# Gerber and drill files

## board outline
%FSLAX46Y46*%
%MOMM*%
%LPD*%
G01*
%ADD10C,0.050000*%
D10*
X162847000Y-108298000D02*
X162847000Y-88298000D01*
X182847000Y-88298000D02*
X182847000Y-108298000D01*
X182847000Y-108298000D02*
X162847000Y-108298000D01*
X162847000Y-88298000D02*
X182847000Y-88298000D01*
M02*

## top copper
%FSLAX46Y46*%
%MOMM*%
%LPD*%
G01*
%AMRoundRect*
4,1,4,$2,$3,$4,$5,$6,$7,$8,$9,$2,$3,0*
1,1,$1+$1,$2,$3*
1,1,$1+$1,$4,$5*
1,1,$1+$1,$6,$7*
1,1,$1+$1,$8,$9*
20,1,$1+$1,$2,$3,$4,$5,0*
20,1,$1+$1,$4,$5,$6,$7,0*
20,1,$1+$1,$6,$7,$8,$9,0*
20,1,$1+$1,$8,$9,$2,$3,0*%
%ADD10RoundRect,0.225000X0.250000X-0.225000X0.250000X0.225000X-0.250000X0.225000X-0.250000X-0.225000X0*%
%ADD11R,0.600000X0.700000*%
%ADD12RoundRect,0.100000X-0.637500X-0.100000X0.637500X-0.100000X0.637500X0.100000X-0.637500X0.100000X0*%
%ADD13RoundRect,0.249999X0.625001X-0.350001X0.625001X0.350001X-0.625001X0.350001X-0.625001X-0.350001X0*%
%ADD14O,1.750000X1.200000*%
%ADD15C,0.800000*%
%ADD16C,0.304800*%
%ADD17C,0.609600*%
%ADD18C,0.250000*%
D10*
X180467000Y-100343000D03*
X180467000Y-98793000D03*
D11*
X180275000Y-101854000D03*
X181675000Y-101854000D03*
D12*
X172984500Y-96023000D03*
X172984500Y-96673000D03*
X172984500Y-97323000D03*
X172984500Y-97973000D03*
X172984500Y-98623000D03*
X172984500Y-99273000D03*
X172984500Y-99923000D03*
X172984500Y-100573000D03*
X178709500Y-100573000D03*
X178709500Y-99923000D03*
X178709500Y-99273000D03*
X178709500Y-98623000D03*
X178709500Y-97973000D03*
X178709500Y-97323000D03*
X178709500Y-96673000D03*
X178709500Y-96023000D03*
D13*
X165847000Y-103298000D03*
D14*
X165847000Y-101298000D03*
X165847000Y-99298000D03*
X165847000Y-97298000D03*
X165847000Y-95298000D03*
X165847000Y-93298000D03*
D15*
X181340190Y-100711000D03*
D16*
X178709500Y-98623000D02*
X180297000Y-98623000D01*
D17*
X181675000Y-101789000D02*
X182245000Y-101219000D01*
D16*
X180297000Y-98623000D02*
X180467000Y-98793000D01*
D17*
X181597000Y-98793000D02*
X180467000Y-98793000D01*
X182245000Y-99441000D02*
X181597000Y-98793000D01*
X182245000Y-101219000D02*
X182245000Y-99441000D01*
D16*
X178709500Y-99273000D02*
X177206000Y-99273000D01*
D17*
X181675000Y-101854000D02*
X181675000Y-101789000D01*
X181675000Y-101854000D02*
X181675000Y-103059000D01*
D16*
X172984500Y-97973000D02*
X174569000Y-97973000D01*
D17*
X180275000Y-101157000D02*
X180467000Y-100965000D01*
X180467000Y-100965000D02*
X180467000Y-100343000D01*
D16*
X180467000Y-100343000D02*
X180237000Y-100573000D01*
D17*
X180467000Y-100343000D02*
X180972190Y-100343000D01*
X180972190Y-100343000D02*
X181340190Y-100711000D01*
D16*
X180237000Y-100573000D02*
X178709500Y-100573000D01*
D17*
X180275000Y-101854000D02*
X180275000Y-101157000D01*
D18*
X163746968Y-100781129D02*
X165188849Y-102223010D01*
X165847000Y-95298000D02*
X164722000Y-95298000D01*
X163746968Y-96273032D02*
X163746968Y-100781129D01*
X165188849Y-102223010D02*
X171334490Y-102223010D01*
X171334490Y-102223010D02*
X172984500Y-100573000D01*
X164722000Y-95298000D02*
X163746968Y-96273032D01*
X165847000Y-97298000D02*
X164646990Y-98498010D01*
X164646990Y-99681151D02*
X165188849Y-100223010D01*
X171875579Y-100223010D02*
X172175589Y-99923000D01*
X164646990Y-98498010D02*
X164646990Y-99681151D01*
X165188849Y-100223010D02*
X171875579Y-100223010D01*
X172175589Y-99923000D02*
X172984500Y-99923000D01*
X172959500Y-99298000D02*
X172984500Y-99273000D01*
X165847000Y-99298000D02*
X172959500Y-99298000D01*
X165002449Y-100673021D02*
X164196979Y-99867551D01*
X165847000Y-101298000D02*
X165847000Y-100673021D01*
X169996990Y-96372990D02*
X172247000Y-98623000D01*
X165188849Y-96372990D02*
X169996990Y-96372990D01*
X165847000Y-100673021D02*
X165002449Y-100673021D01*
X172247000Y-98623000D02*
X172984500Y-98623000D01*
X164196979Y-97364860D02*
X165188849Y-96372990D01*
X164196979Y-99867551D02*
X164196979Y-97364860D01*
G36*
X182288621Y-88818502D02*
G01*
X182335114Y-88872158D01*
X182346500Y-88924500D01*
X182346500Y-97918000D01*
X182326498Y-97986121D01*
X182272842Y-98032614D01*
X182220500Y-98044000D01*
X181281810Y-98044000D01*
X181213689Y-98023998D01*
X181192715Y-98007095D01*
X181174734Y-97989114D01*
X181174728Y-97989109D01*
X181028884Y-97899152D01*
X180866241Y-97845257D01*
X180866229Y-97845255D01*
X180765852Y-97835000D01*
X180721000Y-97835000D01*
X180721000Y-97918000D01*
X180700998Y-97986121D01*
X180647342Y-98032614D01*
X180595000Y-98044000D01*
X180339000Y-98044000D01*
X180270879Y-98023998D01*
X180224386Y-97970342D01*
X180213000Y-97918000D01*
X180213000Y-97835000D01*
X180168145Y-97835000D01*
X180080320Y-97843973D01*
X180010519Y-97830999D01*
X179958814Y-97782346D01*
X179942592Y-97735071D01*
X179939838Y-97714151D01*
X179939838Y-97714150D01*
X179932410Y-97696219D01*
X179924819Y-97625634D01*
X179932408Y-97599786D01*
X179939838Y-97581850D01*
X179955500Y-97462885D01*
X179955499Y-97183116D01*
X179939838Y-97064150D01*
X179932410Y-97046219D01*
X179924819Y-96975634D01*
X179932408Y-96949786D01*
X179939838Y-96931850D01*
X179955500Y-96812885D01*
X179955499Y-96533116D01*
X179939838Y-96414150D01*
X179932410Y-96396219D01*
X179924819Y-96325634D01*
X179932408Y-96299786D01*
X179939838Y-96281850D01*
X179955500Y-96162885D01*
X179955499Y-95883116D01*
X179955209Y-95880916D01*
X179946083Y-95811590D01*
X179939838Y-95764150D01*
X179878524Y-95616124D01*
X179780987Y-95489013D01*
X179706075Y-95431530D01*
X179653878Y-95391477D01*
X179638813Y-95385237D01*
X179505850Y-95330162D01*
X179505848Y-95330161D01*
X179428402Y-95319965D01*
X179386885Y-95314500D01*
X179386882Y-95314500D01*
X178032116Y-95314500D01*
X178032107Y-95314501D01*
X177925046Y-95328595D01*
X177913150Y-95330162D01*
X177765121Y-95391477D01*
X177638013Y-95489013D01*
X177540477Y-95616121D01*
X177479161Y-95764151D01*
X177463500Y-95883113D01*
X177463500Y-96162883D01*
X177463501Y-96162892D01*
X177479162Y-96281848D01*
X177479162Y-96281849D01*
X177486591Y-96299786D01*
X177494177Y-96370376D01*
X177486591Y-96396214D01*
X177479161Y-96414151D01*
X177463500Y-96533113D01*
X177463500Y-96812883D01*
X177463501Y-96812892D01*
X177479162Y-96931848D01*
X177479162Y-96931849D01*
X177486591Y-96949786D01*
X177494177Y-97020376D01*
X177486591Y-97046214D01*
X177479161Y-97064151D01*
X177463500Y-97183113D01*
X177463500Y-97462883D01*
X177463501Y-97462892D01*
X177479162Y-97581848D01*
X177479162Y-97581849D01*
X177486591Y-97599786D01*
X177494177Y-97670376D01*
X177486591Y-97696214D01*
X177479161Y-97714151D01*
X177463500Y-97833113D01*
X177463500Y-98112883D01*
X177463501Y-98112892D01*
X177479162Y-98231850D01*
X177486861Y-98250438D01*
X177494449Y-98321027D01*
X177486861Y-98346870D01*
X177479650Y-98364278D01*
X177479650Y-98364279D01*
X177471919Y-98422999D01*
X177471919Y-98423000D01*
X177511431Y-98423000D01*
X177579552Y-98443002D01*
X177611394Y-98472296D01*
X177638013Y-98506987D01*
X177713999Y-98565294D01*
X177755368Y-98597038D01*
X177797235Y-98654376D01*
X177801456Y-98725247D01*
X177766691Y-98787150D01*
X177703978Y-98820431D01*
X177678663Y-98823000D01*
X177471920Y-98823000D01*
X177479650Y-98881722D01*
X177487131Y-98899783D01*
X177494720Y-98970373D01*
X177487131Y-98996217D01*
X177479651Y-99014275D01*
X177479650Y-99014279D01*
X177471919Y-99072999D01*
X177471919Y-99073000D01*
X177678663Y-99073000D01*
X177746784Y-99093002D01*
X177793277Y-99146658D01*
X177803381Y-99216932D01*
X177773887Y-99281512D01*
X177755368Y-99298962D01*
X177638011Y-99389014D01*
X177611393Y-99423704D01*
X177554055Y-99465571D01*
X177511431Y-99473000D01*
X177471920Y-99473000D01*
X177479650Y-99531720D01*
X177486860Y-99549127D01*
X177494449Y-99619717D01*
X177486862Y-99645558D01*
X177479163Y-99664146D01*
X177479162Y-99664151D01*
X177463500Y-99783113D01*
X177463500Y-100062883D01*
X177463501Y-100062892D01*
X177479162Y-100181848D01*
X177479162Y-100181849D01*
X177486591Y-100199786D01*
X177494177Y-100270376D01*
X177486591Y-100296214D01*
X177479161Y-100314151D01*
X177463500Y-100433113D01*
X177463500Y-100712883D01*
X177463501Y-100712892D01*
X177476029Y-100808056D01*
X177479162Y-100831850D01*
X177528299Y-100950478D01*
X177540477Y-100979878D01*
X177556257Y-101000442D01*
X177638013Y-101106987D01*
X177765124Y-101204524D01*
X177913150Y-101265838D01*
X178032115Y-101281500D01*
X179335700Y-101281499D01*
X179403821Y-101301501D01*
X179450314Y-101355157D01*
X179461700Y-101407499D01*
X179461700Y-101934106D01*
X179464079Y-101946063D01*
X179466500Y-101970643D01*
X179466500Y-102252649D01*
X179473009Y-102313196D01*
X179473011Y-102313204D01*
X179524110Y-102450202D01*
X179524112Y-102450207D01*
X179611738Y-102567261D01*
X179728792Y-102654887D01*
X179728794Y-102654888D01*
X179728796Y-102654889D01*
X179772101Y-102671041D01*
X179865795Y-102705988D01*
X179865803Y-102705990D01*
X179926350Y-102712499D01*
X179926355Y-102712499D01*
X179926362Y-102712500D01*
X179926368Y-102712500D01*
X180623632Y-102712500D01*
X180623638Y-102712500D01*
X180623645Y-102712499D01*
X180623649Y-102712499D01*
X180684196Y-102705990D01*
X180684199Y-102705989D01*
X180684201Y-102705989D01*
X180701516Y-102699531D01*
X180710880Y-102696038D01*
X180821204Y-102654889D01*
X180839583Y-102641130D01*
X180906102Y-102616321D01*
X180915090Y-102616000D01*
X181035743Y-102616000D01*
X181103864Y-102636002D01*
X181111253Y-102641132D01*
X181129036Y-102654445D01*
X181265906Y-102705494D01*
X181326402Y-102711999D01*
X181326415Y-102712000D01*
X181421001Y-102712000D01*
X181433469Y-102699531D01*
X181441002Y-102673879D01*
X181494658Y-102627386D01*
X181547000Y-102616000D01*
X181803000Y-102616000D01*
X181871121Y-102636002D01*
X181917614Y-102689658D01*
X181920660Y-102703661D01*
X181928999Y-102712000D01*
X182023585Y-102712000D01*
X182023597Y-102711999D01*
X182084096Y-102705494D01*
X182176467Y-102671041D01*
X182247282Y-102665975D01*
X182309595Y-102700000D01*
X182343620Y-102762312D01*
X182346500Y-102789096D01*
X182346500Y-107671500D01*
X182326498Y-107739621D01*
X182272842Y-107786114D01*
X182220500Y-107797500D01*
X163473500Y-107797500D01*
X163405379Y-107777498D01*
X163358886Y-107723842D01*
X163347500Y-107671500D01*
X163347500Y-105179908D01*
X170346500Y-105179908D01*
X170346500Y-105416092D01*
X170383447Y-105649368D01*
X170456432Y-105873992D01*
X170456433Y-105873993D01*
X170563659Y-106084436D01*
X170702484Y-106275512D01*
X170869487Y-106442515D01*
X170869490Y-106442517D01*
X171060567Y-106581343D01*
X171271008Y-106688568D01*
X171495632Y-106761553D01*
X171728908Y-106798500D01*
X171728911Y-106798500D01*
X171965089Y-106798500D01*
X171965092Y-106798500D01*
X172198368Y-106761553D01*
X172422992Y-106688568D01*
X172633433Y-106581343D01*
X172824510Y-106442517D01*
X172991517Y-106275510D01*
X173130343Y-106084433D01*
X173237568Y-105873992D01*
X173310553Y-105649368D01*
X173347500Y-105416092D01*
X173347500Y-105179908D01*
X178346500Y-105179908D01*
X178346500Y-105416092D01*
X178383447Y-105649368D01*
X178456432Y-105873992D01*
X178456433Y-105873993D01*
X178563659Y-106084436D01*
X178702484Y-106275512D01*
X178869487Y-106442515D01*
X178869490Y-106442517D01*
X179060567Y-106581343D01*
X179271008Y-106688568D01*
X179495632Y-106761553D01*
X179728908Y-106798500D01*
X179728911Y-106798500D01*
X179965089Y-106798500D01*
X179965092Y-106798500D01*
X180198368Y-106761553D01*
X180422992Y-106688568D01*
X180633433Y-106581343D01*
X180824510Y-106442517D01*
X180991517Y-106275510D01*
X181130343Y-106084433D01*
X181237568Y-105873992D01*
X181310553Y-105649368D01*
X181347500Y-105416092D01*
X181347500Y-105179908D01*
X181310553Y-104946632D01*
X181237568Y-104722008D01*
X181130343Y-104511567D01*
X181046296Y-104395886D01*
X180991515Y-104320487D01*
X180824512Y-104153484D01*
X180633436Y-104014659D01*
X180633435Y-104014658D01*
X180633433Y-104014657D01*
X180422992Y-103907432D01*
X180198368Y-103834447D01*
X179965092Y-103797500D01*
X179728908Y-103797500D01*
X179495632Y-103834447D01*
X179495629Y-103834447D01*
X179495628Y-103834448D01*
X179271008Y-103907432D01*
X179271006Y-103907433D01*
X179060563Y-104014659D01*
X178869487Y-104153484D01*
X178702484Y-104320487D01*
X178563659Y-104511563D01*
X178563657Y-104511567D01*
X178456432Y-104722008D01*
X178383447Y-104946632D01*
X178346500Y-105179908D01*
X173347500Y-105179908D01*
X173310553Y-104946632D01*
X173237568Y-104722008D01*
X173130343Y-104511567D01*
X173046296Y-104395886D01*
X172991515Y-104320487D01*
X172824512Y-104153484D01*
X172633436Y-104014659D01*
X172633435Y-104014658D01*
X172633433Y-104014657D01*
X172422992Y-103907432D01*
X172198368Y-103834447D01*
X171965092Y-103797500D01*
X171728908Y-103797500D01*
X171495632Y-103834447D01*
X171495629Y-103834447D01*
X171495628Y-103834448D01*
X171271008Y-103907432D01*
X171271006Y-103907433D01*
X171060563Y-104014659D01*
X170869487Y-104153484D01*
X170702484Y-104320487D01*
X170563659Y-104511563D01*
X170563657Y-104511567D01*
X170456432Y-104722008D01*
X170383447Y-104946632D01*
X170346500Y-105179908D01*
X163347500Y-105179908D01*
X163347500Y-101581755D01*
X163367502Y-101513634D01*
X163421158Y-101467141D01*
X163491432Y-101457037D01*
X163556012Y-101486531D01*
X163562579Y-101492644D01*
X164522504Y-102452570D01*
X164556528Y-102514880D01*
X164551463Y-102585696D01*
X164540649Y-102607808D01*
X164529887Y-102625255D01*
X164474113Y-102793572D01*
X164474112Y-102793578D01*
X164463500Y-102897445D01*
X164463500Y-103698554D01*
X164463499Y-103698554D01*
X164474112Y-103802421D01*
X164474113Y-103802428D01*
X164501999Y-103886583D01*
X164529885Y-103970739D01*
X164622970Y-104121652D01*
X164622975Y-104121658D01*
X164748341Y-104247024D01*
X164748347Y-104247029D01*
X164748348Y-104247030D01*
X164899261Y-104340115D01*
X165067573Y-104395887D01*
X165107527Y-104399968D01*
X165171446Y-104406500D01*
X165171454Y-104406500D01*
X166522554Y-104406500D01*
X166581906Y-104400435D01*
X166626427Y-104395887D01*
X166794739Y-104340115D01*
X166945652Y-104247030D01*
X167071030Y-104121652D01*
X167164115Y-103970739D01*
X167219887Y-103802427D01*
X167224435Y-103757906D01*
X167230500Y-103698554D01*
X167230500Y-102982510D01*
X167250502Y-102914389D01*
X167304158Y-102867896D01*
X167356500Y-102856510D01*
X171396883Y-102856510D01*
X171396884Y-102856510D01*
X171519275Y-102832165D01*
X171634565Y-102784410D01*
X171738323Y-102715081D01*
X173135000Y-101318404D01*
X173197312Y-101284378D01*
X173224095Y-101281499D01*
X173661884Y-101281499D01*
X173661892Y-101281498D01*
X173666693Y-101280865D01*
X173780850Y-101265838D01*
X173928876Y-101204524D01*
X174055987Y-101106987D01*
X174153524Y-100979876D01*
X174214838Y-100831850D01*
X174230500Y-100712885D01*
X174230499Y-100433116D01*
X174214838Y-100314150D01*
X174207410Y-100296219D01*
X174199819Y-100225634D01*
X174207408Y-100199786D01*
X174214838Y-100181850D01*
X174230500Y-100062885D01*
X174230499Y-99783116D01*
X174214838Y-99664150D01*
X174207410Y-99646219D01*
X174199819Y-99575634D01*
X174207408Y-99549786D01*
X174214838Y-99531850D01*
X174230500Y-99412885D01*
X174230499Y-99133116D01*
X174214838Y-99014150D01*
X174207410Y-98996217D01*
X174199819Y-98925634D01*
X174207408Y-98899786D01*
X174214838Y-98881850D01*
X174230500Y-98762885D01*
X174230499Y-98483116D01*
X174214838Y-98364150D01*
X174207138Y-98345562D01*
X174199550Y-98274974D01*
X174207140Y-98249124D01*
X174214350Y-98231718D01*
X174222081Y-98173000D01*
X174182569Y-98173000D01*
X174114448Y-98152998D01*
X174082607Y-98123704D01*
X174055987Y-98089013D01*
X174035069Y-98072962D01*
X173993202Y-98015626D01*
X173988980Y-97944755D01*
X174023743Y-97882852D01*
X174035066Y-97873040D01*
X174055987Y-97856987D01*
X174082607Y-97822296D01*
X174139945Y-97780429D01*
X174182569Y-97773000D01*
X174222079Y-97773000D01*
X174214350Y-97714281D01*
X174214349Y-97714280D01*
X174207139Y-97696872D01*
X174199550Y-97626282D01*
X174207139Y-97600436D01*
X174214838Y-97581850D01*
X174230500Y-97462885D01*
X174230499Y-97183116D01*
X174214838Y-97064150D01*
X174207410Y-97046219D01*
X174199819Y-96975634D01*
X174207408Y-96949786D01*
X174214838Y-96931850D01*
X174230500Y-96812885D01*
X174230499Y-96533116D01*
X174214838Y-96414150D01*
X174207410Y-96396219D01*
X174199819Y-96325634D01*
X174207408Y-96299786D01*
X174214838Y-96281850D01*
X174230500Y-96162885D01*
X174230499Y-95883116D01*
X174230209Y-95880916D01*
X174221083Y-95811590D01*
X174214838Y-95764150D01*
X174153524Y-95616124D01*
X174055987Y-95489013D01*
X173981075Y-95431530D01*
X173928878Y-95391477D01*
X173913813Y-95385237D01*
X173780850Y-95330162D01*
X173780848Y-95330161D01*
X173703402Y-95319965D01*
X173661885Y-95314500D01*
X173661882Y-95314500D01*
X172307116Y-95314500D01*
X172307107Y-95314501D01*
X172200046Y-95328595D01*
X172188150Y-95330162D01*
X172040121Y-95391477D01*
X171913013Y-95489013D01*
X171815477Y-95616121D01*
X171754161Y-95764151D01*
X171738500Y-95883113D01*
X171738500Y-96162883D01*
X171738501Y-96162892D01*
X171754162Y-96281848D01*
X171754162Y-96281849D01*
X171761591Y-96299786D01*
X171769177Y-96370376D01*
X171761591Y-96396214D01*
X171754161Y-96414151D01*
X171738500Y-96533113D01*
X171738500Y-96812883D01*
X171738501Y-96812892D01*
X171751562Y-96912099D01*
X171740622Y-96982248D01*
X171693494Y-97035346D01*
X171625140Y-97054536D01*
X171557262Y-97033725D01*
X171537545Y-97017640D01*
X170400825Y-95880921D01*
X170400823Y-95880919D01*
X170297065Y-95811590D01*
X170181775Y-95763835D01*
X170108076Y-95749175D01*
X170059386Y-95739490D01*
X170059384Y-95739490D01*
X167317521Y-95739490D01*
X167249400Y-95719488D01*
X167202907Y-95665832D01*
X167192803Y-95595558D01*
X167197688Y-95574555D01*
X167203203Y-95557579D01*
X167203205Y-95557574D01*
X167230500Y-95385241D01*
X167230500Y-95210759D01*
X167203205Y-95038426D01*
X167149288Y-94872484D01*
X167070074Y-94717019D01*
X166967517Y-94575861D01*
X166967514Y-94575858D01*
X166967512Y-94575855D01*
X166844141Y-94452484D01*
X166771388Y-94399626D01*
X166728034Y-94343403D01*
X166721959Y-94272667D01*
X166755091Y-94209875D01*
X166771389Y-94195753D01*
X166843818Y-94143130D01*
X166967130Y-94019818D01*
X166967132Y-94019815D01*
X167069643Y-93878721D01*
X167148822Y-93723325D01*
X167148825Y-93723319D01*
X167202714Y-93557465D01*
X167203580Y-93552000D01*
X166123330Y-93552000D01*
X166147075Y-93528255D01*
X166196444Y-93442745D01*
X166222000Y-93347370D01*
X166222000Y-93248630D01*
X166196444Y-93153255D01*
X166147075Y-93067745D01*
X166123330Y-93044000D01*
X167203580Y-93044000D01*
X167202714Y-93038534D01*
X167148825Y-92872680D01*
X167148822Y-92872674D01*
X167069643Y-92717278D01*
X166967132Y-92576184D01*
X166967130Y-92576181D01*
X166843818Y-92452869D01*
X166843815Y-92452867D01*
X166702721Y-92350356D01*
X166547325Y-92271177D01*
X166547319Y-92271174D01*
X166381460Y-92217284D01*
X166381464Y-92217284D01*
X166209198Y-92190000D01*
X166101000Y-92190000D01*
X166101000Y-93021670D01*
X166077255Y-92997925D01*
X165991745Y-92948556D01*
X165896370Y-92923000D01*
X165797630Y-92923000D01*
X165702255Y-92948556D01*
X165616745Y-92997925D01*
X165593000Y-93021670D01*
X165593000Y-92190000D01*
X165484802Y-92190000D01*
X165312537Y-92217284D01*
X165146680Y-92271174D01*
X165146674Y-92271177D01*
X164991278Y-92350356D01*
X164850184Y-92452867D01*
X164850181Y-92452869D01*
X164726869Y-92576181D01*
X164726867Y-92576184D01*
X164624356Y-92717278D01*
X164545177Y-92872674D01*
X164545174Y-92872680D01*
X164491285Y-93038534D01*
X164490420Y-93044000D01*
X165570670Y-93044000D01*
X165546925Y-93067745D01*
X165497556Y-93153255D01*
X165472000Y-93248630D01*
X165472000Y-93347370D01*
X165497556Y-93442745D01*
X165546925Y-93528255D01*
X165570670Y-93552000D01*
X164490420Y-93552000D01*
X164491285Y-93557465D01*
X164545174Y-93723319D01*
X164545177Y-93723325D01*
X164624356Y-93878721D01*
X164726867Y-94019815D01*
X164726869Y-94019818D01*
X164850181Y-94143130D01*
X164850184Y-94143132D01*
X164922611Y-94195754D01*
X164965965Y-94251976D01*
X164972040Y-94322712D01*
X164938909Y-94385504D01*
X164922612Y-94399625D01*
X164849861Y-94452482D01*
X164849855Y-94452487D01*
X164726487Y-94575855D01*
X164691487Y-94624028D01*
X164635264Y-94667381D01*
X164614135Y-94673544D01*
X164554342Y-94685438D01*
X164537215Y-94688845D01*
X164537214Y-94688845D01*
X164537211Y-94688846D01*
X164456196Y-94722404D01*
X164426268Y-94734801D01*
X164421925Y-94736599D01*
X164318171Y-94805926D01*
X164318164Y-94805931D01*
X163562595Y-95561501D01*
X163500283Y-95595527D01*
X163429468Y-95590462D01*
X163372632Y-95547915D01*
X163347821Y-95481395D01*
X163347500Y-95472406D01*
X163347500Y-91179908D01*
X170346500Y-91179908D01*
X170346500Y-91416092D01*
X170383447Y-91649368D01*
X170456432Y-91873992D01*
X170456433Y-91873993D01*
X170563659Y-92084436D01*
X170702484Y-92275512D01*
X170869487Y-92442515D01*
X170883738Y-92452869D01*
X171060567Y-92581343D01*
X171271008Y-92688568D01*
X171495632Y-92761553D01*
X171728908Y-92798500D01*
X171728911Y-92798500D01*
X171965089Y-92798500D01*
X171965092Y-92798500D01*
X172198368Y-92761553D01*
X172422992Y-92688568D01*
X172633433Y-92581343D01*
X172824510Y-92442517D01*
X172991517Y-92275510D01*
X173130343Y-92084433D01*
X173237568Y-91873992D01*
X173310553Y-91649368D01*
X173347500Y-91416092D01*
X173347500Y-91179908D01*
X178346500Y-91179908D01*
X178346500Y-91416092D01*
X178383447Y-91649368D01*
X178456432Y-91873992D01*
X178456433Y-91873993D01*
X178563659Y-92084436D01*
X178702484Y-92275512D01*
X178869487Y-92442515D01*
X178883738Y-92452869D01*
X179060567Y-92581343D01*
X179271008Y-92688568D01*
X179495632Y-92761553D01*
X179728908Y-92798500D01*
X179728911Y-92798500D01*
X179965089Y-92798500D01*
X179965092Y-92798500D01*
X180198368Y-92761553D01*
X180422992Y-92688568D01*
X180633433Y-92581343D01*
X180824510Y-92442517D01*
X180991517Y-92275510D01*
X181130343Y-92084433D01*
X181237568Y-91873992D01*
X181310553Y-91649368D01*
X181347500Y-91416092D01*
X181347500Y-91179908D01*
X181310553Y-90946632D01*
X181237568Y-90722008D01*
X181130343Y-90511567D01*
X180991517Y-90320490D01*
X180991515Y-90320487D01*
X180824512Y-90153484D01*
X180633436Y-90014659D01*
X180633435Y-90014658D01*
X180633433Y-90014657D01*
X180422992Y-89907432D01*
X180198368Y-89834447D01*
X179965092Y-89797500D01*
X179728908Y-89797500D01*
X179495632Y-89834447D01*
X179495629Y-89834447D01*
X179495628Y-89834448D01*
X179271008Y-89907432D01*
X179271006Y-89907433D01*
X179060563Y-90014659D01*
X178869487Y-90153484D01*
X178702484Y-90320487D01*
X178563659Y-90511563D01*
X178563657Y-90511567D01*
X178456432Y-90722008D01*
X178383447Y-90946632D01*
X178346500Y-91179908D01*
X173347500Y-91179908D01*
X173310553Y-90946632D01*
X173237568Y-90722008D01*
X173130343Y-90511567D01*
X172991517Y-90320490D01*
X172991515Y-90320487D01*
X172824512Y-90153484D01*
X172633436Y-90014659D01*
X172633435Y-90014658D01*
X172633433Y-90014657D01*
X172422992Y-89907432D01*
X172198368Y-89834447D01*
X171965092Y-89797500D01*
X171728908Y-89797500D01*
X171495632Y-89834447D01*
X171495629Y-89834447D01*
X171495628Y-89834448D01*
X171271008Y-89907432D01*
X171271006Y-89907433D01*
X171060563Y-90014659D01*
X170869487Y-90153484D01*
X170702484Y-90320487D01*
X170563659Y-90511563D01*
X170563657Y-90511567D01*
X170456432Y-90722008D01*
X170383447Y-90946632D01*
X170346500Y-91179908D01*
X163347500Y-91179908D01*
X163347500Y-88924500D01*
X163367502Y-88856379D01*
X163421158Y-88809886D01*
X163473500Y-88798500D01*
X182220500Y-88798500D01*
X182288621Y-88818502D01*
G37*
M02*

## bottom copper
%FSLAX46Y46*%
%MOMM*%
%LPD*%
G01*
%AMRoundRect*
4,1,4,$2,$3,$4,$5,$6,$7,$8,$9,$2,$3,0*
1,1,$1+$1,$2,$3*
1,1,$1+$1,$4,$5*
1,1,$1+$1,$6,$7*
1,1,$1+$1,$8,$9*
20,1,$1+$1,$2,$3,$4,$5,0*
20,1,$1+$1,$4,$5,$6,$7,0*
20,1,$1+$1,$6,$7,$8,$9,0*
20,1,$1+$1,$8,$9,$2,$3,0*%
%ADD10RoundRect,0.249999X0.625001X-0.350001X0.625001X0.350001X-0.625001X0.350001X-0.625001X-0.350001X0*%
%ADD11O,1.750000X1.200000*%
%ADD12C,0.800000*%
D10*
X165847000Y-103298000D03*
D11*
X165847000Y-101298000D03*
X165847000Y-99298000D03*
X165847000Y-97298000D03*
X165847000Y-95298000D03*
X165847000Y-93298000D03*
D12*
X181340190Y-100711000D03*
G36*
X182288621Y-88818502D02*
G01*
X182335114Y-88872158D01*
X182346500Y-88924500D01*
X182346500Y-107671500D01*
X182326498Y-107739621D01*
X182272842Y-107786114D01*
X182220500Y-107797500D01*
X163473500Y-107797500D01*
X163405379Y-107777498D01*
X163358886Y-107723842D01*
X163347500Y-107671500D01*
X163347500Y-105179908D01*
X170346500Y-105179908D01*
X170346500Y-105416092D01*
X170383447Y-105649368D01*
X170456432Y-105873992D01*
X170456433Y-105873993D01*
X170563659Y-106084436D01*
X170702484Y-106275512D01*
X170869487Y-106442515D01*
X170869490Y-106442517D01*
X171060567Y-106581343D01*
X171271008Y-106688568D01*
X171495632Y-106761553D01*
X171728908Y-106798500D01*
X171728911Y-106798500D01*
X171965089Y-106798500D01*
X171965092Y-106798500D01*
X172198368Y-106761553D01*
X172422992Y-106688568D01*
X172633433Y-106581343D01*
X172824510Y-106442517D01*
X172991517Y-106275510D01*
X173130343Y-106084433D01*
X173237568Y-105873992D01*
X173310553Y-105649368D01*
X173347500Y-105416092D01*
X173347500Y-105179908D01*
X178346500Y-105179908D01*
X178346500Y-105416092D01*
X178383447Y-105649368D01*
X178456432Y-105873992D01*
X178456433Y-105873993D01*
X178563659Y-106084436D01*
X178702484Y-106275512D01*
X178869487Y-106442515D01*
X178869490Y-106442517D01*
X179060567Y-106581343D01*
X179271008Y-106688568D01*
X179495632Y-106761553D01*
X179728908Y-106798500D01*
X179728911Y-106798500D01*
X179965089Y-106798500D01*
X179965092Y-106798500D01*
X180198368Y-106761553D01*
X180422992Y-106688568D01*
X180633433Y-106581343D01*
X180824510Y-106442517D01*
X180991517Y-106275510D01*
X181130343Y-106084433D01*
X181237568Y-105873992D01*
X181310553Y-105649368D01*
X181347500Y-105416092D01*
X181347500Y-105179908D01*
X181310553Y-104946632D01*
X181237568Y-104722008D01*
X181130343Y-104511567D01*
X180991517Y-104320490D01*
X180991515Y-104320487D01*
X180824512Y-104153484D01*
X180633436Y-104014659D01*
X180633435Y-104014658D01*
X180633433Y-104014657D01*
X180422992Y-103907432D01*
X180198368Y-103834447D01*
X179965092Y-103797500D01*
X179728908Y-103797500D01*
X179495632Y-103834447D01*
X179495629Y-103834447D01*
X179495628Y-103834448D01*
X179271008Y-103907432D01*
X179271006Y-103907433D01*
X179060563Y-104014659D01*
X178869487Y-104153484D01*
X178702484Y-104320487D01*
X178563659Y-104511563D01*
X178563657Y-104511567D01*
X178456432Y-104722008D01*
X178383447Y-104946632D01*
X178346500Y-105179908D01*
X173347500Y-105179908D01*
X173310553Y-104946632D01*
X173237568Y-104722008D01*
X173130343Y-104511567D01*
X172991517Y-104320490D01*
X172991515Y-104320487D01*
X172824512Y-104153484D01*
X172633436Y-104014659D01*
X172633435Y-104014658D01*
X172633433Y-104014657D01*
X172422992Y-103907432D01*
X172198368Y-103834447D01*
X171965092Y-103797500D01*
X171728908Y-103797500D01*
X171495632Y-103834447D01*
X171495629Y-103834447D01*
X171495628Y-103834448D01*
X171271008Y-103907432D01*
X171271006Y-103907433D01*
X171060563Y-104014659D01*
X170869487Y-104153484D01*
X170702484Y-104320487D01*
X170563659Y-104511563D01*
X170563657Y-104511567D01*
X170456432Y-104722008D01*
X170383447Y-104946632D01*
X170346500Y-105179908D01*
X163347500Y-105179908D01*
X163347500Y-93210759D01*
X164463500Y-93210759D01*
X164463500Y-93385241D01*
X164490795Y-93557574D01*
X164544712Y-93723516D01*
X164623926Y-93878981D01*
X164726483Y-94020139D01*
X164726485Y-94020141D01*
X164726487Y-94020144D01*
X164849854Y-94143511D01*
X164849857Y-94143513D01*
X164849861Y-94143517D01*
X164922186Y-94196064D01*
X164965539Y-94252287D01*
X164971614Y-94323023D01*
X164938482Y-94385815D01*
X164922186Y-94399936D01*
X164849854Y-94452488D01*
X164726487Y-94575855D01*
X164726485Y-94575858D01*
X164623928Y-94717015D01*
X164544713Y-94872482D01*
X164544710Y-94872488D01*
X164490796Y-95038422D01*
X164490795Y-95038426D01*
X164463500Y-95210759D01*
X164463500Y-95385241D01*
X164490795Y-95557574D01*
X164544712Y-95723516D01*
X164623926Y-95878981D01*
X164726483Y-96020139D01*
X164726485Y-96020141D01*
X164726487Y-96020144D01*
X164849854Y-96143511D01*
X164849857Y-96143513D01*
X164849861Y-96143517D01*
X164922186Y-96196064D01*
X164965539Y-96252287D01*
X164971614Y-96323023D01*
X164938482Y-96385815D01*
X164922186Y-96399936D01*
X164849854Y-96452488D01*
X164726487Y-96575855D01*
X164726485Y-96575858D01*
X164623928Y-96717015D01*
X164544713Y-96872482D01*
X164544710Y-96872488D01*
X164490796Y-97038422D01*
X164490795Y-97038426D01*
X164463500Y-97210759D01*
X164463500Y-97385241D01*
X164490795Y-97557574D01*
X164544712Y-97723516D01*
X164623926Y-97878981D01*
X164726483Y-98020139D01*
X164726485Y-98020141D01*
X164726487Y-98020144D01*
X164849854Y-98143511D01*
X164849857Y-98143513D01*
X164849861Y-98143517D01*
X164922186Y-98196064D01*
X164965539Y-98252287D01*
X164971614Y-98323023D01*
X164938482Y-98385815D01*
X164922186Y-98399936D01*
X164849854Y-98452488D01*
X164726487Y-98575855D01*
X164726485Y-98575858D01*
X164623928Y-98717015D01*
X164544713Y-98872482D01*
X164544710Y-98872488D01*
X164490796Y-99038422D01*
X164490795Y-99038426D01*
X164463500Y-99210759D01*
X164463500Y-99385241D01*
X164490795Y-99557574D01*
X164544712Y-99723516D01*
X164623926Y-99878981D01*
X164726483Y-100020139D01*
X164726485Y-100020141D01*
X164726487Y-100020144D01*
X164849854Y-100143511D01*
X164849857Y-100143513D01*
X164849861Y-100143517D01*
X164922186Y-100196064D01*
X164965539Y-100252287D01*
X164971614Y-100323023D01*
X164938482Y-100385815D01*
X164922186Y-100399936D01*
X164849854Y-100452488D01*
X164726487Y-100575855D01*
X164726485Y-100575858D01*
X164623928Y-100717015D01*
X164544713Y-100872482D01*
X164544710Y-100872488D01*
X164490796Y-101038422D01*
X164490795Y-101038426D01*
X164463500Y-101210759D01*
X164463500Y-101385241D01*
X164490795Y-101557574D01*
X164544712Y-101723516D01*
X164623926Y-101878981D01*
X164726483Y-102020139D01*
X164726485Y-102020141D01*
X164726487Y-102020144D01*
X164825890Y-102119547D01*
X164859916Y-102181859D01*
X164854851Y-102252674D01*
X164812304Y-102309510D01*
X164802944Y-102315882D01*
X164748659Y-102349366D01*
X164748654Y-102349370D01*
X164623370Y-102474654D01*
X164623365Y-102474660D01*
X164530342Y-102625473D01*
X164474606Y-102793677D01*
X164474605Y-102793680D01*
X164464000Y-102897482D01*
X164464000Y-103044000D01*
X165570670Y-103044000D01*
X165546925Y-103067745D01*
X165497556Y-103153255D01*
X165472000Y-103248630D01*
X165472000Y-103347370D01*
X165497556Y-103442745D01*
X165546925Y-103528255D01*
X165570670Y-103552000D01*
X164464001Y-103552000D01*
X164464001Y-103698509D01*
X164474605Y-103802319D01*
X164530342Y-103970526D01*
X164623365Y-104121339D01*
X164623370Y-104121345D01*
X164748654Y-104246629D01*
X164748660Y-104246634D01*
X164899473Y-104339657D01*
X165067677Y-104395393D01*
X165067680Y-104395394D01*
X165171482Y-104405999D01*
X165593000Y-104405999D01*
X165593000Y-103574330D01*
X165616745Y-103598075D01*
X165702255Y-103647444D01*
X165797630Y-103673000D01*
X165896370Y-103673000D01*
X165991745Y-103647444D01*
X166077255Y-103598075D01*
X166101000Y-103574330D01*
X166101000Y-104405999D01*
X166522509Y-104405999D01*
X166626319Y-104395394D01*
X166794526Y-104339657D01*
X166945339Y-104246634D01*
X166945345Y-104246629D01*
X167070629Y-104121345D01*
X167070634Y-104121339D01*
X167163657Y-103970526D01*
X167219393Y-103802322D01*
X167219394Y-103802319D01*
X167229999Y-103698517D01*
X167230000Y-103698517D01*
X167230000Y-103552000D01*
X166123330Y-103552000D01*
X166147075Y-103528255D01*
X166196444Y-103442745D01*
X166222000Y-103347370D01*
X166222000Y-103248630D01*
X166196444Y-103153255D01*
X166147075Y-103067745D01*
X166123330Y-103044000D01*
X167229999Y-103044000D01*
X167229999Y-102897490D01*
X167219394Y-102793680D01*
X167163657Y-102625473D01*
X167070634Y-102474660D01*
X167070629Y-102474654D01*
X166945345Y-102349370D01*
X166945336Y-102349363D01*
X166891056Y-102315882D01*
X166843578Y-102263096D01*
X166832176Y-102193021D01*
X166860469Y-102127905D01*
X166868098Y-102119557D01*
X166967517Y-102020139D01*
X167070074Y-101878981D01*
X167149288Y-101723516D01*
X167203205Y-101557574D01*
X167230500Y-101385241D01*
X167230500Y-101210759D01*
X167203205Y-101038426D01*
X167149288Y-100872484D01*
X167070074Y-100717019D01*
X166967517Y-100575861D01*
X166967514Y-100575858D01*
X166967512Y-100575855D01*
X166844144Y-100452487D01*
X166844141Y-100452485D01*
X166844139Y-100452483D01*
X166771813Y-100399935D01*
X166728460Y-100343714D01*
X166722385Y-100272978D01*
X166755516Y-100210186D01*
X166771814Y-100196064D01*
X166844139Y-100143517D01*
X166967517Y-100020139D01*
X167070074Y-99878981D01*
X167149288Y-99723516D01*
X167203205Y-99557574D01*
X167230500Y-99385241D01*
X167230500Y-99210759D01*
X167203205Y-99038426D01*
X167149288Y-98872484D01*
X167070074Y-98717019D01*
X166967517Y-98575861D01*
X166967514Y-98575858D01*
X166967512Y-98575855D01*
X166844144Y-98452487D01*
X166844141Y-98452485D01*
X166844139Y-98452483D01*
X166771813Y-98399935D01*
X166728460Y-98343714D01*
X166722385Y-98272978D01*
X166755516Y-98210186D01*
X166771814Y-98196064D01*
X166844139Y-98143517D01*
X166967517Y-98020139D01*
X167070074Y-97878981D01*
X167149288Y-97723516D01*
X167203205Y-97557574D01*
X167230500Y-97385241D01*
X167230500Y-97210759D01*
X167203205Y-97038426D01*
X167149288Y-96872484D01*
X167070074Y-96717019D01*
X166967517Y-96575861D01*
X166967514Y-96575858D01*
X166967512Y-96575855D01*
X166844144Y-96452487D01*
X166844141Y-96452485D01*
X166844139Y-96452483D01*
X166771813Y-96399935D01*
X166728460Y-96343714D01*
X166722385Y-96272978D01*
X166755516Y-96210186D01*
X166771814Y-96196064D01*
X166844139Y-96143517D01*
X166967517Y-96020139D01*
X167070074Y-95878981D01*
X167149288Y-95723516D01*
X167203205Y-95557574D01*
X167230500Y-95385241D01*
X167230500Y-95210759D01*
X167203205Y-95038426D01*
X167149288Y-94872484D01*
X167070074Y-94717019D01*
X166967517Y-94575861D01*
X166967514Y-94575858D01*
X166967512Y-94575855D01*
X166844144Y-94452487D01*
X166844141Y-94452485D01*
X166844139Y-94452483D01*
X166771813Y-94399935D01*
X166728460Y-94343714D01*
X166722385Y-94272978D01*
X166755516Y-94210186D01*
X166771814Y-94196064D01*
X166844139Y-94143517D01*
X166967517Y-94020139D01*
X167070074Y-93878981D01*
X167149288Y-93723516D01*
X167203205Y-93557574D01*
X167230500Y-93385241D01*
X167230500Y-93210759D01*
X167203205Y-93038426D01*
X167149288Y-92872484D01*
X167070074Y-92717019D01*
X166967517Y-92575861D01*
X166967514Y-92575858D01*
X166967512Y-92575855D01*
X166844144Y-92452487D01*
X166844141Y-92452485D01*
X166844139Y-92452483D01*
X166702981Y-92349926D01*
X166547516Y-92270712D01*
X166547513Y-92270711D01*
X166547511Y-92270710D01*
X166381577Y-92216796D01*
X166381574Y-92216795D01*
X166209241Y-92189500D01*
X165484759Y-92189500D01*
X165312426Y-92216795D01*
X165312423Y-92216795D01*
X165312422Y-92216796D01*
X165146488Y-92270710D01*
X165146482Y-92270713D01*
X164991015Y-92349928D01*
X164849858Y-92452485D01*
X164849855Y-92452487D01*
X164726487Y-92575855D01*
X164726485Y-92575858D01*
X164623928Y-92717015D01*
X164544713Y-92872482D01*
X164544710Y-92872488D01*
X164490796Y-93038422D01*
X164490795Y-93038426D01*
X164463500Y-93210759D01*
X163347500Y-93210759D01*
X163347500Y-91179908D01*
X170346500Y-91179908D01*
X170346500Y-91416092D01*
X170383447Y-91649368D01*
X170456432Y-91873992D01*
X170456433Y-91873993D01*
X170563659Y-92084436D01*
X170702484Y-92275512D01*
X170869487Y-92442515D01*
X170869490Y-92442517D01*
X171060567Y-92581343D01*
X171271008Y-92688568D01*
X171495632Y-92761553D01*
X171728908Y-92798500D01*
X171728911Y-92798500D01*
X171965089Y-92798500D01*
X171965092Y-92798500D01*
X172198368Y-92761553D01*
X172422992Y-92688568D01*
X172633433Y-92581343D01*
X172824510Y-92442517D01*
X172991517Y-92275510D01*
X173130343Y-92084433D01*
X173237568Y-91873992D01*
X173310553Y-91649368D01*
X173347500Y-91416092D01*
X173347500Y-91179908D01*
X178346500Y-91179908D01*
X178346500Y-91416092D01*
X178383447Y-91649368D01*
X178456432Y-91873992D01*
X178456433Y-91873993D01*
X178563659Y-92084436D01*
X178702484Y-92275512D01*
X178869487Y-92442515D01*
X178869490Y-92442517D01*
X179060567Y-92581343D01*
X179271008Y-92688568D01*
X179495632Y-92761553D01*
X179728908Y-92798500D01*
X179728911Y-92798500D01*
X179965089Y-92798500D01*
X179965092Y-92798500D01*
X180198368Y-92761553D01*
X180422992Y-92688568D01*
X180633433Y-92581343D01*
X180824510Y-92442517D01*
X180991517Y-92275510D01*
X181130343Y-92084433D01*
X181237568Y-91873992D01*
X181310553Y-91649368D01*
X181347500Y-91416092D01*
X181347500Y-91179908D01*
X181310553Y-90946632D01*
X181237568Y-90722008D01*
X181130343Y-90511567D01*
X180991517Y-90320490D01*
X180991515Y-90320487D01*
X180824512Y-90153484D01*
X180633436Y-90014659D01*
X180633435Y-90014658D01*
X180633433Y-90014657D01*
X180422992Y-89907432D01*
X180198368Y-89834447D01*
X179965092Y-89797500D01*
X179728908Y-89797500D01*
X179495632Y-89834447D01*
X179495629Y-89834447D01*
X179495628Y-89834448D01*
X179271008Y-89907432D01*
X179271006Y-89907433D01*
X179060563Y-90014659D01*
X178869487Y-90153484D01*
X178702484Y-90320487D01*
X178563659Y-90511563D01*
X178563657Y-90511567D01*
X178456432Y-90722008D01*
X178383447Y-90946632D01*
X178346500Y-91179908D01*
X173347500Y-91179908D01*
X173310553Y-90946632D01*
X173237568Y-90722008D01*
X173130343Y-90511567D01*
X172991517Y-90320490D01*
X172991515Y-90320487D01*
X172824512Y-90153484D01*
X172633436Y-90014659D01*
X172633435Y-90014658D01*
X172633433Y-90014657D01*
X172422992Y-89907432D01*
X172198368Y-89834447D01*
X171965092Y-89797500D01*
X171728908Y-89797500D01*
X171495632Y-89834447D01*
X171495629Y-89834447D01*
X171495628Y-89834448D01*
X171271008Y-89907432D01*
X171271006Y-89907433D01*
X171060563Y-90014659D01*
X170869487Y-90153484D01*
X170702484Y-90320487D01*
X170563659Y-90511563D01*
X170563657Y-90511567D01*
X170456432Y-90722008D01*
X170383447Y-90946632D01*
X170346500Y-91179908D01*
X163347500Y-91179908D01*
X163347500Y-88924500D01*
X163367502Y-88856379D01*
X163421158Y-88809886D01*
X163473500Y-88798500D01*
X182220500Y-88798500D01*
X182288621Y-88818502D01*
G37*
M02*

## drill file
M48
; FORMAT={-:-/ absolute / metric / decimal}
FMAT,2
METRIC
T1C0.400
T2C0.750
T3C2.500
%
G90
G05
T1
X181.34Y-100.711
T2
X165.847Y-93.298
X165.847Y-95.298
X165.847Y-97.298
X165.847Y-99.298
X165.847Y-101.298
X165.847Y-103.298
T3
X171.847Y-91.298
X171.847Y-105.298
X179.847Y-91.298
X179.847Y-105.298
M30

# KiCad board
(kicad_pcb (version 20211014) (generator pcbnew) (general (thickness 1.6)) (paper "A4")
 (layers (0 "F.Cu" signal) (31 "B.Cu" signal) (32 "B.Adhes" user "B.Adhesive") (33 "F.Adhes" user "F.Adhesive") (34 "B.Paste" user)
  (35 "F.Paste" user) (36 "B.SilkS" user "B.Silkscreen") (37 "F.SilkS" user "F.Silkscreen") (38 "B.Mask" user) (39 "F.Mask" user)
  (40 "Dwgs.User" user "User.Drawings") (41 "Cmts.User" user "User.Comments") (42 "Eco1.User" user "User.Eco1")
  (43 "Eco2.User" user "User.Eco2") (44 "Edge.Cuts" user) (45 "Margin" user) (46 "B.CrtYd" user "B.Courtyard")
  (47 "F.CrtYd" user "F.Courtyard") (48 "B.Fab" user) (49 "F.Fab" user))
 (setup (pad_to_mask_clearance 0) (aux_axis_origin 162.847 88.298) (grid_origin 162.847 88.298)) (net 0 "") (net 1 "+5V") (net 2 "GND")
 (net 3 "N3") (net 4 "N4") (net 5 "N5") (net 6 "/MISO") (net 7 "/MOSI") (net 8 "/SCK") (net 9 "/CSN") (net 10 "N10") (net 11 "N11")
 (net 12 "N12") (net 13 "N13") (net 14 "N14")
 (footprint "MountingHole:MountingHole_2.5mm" (layer "F.Cu") (at 179.847 91.298)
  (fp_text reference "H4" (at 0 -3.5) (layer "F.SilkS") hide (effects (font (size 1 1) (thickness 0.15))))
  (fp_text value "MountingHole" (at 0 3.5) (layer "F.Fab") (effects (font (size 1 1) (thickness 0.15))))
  (pad "" np_thru_hole circle locked (at 0 0) (size 2.5 2.5) (drill 2.5) (layers *.Cu *.Mask)))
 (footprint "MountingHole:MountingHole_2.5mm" (layer "F.Cu") (at 179.847 105.298)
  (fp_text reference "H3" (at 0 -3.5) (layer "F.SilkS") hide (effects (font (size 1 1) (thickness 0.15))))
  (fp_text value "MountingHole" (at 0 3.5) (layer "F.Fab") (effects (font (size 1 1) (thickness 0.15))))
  (pad "" np_thru_hole circle locked (at 0 0) (size 2.5 2.5) (drill 2.5) (layers *.Cu *.Mask)))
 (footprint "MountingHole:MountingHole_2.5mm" (layer "F.Cu") (at 171.847 91.298)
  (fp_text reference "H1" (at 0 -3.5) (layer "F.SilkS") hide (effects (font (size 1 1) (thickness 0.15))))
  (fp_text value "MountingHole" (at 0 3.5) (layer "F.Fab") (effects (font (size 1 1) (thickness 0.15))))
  (pad "" np_thru_hole circle locked (at 0 0) (size 2.5 2.5) (drill 2.5) (layers *.Cu *.Mask)))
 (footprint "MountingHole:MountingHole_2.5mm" (layer "F.Cu") (at 171.847 105.298)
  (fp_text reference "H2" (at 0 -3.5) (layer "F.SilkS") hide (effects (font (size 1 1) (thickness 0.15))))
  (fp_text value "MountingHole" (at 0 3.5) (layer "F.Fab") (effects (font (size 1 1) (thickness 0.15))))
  (pad "" np_thru_hole circle locked (at 0 0) (size 2.5 2.5) (drill 2.5) (layers *.Cu *.Mask)))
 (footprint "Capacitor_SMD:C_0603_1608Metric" (layer "F.Cu") (at 180.467 99.568 90)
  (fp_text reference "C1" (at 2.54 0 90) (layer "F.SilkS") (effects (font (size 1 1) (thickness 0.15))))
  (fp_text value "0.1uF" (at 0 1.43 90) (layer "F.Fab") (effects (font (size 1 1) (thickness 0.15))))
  (pad "1" smd roundrect locked (at -0.775 0 90) (size 0.9 0.95) (layers "F.Cu" "F.Paste" "F.Mask") (roundrect_rratio 0.25) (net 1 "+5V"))
  (pad "2" smd roundrect locked (at 0.775 0 90) (size 0.9 0.95) (layers "F.Cu" "F.Paste" "F.Mask") (roundrect_rratio 0.25) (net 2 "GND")))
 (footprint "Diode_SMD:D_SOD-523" (layer "F.Cu") (at 180.975 101.854)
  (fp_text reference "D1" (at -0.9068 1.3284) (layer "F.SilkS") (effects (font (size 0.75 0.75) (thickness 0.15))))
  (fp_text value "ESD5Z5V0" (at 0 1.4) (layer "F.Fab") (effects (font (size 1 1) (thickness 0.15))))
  (pad "1" smd rect locked (at -0.7 0 180) (size 0.6 0.7) (layers "F.Cu" "F.Paste" "F.Mask") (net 1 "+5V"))
  (pad "2" smd rect locked (at 0.7 0 180) (size 0.6 0.7) (layers "F.Cu" "F.Paste" "F.Mask") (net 2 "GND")))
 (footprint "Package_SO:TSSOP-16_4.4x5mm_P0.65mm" (layer "F.Cu") (at 175.847 98.298)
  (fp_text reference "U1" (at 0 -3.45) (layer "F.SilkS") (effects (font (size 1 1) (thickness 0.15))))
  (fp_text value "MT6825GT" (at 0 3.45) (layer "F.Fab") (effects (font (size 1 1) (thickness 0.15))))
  (pad "1" smd roundrect locked (at -2.8625 -2.275) (size 1.475 0.4) (layers "F.Cu" "F.Paste" "F.Mask") (roundrect_rratio 0.25) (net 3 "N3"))
  (pad "2" smd roundrect locked (at -2.8625 -1.625) (size 1.475 0.4) (layers "F.Cu" "F.Paste" "F.Mask") (roundrect_rratio 0.25) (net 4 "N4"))
  (pad "3" smd roundrect locked (at -2.8625 -0.975) (size 1.475 0.4) (layers "F.Cu" "F.Paste" "F.Mask") (roundrect_rratio 0.25) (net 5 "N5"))
  (pad "4" smd roundrect locked (at -2.8625 -0.325) (size 1.475 0.4) (layers "F.Cu" "F.Paste" "F.Mask") (roundrect_rratio 0.25)
   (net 2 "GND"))
  (pad "5" smd roundrect locked (at -2.8625 0.325) (size 1.475 0.4) (layers "F.Cu" "F.Paste" "F.Mask") (roundrect_rratio 0.25)
   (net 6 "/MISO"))
  (pad "6" smd roundrect locked (at -2.8625 0.975) (size 1.475 0.4) (layers "F.Cu" "F.Paste" "F.Mask") (roundrect_rratio 0.25)
   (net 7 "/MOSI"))
  (pad "7" smd roundrect locked (at -2.8625 1.625) (size 1.475 0.4) (layers "F.Cu" "F.Paste" "F.Mask") (roundrect_rratio 0.25)
   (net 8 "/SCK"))
  (pad "8" smd roundrect locked (at -2.8625 2.275) (size 1.475 0.4) (layers "F.Cu" "F.Paste" "F.Mask") (roundrect_rratio 0.25)
   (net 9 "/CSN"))
  (pad "9" smd roundrect locked (at 2.8625 2.275) (size 1.475 0.4) (layers "F.Cu" "F.Paste" "F.Mask") (roundrect_rratio 0.25) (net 1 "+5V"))
  (pad "10" smd roundrect locked (at 2.8625 1.625) (size 1.475 0.4) (layers "F.Cu" "F.Paste" "F.Mask") (roundrect_rratio 0.25)
   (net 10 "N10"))
  (pad "11" smd roundrect locked (at 2.8625 0.975) (size 1.475 0.4) (layers "F.Cu" "F.Paste" "F.Mask") (roundrect_rratio 0.25) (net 2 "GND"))
  (pad "12" smd roundrect locked (at 2.8625 0.325) (size 1.475 0.4) (layers "F.Cu" "F.Paste" "F.Mask") (roundrect_rratio 0.25) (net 2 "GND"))
  (pad "13" smd roundrect locked (at 2.8625 -0.325) (size 1.475 0.4) (layers "F.Cu" "F.Paste" "F.Mask") (roundrect_rratio 0.25)
   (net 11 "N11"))
  (pad "14" smd roundrect locked (at 2.8625 -0.975) (size 1.475 0.4) (layers "F.Cu" "F.Paste" "F.Mask") (roundrect_rratio 0.25)
   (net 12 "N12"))
  (pad "15" smd roundrect locked (at 2.8625 -1.625) (size 1.475 0.4) (layers "F.Cu" "F.Paste" "F.Mask") (roundrect_rratio 0.25)
   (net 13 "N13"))
  (pad "16" smd roundrect locked (at 2.8625 -2.275) (size 1.475 0.4) (layers "F.Cu" "F.Paste" "F.Mask") (roundrect_rratio 0.25)
   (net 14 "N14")))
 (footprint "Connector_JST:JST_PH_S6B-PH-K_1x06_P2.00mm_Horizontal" (layer "B.Cu") (at 165.847 103.298 90)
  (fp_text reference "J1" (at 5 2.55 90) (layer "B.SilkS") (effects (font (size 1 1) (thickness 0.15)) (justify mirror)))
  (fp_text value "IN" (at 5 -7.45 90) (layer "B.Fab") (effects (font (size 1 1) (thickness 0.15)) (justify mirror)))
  (pad "1" thru_hole roundrect locked (at 0 0 90) (size 1.2 1.75) (drill 0.75) (layers *.Cu *.Mask) (roundrect_rratio 0.2083325)
   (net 1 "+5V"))
  (pad "2" thru_hole oval locked (at 2 0 90) (size 1.2 1.75) (drill 0.75) (layers *.Cu *.Mask) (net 6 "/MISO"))
  (pad "3" thru_hole oval locked (at 4 0 90) (size 1.2 1.75) (drill 0.75) (layers *.Cu *.Mask) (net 7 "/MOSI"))
  (pad "4" thru_hole oval locked (at 6 0 90) (size 1.2 1.75) (drill 0.75) (layers *.Cu *.Mask) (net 8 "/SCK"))
  (pad "5" thru_hole oval locked (at 8 0 90) (size 1.2 1.75) (drill 0.75) (layers *.Cu *.Mask) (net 9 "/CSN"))
  (pad "6" thru_hole oval locked (at 10 0 90) (size 1.2 1.75) (drill 0.75) (layers *.Cu *.Mask) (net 2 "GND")))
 (gr_line (start 162.847 108.298) (end 162.847 88.298) (layer "Edge.Cuts") (width 0.05))
 (gr_line (start 182.847 88.298) (end 182.847 108.298) (layer "Edge.Cuts") (width 0.05))
 (gr_line (start 182.847 108.298) (end 162.847 108.298) (layer "Edge.Cuts") (width 0.05))
 (gr_line (start 162.847 88.298) (end 182.847 88.298) (layer "Edge.Cuts") (width 0.05))
 (segment (start 178.7095 98.623) (end 180.297 98.623) (width 0.3048) (layer "F.Cu") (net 2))
 (segment (start 181.675 101.789) (end 182.245 101.219) (width 0.6096) (layer "F.Cu") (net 2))
 (segment (start 180.297 98.623) (end 180.467 98.793) (width 0.3048) (layer "F.Cu") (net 2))
 (segment (start 181.597 98.793) (end 180.467 98.793) (width 0.6096) (layer "F.Cu") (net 2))
 (segment (start 182.245 99.441) (end 181.597 98.793) (width 0.6096) (layer "F.Cu") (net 2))
 (segment (start 182.245 101.219) (end 182.245 99.441) (width 0.6096) (layer "F.Cu") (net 2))
 (segment (start 178.7095 99.273) (end 177.206 99.273) (width 0.3048) (layer "F.Cu") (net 2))
 (segment (start 181.675 101.854) (end 181.675 101.789) (width 0.6096) (layer "F.Cu") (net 2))
 (segment (start 181.675 101.854) (end 181.675 103.059) (width 0.6096) (layer "F.Cu") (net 2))
 (segment (start 172.9845 97.973) (end 174.569 97.973) (width 0.3048) (layer "F.Cu") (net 2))
 (segment (start 180.275 101.157) (end 180.467 100.965) (width 0.6096) (layer "F.Cu") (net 1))
 (segment (start 180.467 100.965) (end 180.467 100.343) (width 0.6096) (layer "F.Cu") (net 1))
 (segment (start 180.467 100.343) (end 180.237 100.573) (width 0.3048) (layer "F.Cu") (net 1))
 (segment (start 180.467 100.343) (end 180.97219 100.343) (width 0.6096) (layer "F.Cu") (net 1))
 (segment (start 180.97219 100.343) (end 181.34019 100.711) (width 0.6096) (layer "F.Cu") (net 1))
 (segment (start 180.237 100.573) (end 178.7095 100.573) (width 0.3048) (layer "F.Cu") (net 1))
 (segment (start 180.275 101.854) (end 180.275 101.157) (width 0.6096) (layer "F.Cu") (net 1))
 (via (at 181.34019 100.711) (size 0.8) (drill 0.4) (layers "F.Cu" "B.Cu") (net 1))
 (segment (start 163.746968 100.781129) (end 165.188849 102.22301) (width 0.25) (layer "F.Cu") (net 9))
 (segment (start 165.847 95.298) (end 164.722 95.298) (width 0.25) (layer "F.Cu") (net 9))
 (segment (start 163.746968 96.273032) (end 163.746968 100.781129) (width 0.25) (layer "F.Cu") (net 9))
 (segment (start 165.188849 102.22301) (end 171.33449 102.22301) (width 0.25) (layer "F.Cu") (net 9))
 (segment (start 171.33449 102.22301) (end 172.9845 100.573) (width 0.25) (layer "F.Cu") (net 9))
 (segment (start 164.722 95.298) (end 163.746968 96.273032) (width 0.25) (layer "F.Cu") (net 9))
 (segment (start 165.847 97.298) (end 164.64699 98.49801) (width 0.25) (layer "F.Cu") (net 8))
 (segment (start 164.64699 99.681151) (end 165.188849 100.22301) (width 0.25) (layer "F.Cu") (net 8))
 (segment (start 171.875579 100.22301) (end 172.175589 99.923) (width 0.25) (layer "F.Cu") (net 8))
 (segment (start 164.64699 98.49801) (end 164.64699 99.681151) (width 0.25) (layer "F.Cu") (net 8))
 (segment (start 165.188849 100.22301) (end 171.875579 100.22301) (width 0.25) (layer "F.Cu") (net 8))
 (segment (start 172.175589 99.923) (end 172.9845 99.923) (width 0.25) (layer "F.Cu") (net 8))
 (segment (start 172.9595 99.298) (end 172.9845 99.273) (width 0.25) (layer "F.Cu") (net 7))
 (segment (start 165.847 99.298) (end 172.9595 99.298) (width 0.25) (layer "F.Cu") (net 7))
 (segment (start 165.002449 100.673021) (end 164.196979 99.867551) (width 0.25) (layer "F.Cu") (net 6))
 (segment (start 165.847 101.298) (end 165.847 100.673021) (width 0.25) (layer "F.Cu") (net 6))
 (segment (start 169.99699 96.37299) (end 172.247 98.623) (width 0.25) (layer "F.Cu") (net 6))
 (segment (start 165.188849 96.37299) (end 169.99699 96.37299) (width 0.25) (layer "F.Cu") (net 6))
 (segment (start 165.847 100.673021) (end 165.002449 100.673021) (width 0.25) (layer "F.Cu") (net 6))
 (segment (start 172.247 98.623) (end 172.9845 98.623) (width 0.25) (layer "F.Cu") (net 6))
 (segment (start 164.196979 97.36486) (end 165.188849 96.37299) (width 0.25) (layer "F.Cu") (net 6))
 (segment (start 164.196979 99.867551) (end 164.196979 97.36486) (width 0.25) (layer "F.Cu") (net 6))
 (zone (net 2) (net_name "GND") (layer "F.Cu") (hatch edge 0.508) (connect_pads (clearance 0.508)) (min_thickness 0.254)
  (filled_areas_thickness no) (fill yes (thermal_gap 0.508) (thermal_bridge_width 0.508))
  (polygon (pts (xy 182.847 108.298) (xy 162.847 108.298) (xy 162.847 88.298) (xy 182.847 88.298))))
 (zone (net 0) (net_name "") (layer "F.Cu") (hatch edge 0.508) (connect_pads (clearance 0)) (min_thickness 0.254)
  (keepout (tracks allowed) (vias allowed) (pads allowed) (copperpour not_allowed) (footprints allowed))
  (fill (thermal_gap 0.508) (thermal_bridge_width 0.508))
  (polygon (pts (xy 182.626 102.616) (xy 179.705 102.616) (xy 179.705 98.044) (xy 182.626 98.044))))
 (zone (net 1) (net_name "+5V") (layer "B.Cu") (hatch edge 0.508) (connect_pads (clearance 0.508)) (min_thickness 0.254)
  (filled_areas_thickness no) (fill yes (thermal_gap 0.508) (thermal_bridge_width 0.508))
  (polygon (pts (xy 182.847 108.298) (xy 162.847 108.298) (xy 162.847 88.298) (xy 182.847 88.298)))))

